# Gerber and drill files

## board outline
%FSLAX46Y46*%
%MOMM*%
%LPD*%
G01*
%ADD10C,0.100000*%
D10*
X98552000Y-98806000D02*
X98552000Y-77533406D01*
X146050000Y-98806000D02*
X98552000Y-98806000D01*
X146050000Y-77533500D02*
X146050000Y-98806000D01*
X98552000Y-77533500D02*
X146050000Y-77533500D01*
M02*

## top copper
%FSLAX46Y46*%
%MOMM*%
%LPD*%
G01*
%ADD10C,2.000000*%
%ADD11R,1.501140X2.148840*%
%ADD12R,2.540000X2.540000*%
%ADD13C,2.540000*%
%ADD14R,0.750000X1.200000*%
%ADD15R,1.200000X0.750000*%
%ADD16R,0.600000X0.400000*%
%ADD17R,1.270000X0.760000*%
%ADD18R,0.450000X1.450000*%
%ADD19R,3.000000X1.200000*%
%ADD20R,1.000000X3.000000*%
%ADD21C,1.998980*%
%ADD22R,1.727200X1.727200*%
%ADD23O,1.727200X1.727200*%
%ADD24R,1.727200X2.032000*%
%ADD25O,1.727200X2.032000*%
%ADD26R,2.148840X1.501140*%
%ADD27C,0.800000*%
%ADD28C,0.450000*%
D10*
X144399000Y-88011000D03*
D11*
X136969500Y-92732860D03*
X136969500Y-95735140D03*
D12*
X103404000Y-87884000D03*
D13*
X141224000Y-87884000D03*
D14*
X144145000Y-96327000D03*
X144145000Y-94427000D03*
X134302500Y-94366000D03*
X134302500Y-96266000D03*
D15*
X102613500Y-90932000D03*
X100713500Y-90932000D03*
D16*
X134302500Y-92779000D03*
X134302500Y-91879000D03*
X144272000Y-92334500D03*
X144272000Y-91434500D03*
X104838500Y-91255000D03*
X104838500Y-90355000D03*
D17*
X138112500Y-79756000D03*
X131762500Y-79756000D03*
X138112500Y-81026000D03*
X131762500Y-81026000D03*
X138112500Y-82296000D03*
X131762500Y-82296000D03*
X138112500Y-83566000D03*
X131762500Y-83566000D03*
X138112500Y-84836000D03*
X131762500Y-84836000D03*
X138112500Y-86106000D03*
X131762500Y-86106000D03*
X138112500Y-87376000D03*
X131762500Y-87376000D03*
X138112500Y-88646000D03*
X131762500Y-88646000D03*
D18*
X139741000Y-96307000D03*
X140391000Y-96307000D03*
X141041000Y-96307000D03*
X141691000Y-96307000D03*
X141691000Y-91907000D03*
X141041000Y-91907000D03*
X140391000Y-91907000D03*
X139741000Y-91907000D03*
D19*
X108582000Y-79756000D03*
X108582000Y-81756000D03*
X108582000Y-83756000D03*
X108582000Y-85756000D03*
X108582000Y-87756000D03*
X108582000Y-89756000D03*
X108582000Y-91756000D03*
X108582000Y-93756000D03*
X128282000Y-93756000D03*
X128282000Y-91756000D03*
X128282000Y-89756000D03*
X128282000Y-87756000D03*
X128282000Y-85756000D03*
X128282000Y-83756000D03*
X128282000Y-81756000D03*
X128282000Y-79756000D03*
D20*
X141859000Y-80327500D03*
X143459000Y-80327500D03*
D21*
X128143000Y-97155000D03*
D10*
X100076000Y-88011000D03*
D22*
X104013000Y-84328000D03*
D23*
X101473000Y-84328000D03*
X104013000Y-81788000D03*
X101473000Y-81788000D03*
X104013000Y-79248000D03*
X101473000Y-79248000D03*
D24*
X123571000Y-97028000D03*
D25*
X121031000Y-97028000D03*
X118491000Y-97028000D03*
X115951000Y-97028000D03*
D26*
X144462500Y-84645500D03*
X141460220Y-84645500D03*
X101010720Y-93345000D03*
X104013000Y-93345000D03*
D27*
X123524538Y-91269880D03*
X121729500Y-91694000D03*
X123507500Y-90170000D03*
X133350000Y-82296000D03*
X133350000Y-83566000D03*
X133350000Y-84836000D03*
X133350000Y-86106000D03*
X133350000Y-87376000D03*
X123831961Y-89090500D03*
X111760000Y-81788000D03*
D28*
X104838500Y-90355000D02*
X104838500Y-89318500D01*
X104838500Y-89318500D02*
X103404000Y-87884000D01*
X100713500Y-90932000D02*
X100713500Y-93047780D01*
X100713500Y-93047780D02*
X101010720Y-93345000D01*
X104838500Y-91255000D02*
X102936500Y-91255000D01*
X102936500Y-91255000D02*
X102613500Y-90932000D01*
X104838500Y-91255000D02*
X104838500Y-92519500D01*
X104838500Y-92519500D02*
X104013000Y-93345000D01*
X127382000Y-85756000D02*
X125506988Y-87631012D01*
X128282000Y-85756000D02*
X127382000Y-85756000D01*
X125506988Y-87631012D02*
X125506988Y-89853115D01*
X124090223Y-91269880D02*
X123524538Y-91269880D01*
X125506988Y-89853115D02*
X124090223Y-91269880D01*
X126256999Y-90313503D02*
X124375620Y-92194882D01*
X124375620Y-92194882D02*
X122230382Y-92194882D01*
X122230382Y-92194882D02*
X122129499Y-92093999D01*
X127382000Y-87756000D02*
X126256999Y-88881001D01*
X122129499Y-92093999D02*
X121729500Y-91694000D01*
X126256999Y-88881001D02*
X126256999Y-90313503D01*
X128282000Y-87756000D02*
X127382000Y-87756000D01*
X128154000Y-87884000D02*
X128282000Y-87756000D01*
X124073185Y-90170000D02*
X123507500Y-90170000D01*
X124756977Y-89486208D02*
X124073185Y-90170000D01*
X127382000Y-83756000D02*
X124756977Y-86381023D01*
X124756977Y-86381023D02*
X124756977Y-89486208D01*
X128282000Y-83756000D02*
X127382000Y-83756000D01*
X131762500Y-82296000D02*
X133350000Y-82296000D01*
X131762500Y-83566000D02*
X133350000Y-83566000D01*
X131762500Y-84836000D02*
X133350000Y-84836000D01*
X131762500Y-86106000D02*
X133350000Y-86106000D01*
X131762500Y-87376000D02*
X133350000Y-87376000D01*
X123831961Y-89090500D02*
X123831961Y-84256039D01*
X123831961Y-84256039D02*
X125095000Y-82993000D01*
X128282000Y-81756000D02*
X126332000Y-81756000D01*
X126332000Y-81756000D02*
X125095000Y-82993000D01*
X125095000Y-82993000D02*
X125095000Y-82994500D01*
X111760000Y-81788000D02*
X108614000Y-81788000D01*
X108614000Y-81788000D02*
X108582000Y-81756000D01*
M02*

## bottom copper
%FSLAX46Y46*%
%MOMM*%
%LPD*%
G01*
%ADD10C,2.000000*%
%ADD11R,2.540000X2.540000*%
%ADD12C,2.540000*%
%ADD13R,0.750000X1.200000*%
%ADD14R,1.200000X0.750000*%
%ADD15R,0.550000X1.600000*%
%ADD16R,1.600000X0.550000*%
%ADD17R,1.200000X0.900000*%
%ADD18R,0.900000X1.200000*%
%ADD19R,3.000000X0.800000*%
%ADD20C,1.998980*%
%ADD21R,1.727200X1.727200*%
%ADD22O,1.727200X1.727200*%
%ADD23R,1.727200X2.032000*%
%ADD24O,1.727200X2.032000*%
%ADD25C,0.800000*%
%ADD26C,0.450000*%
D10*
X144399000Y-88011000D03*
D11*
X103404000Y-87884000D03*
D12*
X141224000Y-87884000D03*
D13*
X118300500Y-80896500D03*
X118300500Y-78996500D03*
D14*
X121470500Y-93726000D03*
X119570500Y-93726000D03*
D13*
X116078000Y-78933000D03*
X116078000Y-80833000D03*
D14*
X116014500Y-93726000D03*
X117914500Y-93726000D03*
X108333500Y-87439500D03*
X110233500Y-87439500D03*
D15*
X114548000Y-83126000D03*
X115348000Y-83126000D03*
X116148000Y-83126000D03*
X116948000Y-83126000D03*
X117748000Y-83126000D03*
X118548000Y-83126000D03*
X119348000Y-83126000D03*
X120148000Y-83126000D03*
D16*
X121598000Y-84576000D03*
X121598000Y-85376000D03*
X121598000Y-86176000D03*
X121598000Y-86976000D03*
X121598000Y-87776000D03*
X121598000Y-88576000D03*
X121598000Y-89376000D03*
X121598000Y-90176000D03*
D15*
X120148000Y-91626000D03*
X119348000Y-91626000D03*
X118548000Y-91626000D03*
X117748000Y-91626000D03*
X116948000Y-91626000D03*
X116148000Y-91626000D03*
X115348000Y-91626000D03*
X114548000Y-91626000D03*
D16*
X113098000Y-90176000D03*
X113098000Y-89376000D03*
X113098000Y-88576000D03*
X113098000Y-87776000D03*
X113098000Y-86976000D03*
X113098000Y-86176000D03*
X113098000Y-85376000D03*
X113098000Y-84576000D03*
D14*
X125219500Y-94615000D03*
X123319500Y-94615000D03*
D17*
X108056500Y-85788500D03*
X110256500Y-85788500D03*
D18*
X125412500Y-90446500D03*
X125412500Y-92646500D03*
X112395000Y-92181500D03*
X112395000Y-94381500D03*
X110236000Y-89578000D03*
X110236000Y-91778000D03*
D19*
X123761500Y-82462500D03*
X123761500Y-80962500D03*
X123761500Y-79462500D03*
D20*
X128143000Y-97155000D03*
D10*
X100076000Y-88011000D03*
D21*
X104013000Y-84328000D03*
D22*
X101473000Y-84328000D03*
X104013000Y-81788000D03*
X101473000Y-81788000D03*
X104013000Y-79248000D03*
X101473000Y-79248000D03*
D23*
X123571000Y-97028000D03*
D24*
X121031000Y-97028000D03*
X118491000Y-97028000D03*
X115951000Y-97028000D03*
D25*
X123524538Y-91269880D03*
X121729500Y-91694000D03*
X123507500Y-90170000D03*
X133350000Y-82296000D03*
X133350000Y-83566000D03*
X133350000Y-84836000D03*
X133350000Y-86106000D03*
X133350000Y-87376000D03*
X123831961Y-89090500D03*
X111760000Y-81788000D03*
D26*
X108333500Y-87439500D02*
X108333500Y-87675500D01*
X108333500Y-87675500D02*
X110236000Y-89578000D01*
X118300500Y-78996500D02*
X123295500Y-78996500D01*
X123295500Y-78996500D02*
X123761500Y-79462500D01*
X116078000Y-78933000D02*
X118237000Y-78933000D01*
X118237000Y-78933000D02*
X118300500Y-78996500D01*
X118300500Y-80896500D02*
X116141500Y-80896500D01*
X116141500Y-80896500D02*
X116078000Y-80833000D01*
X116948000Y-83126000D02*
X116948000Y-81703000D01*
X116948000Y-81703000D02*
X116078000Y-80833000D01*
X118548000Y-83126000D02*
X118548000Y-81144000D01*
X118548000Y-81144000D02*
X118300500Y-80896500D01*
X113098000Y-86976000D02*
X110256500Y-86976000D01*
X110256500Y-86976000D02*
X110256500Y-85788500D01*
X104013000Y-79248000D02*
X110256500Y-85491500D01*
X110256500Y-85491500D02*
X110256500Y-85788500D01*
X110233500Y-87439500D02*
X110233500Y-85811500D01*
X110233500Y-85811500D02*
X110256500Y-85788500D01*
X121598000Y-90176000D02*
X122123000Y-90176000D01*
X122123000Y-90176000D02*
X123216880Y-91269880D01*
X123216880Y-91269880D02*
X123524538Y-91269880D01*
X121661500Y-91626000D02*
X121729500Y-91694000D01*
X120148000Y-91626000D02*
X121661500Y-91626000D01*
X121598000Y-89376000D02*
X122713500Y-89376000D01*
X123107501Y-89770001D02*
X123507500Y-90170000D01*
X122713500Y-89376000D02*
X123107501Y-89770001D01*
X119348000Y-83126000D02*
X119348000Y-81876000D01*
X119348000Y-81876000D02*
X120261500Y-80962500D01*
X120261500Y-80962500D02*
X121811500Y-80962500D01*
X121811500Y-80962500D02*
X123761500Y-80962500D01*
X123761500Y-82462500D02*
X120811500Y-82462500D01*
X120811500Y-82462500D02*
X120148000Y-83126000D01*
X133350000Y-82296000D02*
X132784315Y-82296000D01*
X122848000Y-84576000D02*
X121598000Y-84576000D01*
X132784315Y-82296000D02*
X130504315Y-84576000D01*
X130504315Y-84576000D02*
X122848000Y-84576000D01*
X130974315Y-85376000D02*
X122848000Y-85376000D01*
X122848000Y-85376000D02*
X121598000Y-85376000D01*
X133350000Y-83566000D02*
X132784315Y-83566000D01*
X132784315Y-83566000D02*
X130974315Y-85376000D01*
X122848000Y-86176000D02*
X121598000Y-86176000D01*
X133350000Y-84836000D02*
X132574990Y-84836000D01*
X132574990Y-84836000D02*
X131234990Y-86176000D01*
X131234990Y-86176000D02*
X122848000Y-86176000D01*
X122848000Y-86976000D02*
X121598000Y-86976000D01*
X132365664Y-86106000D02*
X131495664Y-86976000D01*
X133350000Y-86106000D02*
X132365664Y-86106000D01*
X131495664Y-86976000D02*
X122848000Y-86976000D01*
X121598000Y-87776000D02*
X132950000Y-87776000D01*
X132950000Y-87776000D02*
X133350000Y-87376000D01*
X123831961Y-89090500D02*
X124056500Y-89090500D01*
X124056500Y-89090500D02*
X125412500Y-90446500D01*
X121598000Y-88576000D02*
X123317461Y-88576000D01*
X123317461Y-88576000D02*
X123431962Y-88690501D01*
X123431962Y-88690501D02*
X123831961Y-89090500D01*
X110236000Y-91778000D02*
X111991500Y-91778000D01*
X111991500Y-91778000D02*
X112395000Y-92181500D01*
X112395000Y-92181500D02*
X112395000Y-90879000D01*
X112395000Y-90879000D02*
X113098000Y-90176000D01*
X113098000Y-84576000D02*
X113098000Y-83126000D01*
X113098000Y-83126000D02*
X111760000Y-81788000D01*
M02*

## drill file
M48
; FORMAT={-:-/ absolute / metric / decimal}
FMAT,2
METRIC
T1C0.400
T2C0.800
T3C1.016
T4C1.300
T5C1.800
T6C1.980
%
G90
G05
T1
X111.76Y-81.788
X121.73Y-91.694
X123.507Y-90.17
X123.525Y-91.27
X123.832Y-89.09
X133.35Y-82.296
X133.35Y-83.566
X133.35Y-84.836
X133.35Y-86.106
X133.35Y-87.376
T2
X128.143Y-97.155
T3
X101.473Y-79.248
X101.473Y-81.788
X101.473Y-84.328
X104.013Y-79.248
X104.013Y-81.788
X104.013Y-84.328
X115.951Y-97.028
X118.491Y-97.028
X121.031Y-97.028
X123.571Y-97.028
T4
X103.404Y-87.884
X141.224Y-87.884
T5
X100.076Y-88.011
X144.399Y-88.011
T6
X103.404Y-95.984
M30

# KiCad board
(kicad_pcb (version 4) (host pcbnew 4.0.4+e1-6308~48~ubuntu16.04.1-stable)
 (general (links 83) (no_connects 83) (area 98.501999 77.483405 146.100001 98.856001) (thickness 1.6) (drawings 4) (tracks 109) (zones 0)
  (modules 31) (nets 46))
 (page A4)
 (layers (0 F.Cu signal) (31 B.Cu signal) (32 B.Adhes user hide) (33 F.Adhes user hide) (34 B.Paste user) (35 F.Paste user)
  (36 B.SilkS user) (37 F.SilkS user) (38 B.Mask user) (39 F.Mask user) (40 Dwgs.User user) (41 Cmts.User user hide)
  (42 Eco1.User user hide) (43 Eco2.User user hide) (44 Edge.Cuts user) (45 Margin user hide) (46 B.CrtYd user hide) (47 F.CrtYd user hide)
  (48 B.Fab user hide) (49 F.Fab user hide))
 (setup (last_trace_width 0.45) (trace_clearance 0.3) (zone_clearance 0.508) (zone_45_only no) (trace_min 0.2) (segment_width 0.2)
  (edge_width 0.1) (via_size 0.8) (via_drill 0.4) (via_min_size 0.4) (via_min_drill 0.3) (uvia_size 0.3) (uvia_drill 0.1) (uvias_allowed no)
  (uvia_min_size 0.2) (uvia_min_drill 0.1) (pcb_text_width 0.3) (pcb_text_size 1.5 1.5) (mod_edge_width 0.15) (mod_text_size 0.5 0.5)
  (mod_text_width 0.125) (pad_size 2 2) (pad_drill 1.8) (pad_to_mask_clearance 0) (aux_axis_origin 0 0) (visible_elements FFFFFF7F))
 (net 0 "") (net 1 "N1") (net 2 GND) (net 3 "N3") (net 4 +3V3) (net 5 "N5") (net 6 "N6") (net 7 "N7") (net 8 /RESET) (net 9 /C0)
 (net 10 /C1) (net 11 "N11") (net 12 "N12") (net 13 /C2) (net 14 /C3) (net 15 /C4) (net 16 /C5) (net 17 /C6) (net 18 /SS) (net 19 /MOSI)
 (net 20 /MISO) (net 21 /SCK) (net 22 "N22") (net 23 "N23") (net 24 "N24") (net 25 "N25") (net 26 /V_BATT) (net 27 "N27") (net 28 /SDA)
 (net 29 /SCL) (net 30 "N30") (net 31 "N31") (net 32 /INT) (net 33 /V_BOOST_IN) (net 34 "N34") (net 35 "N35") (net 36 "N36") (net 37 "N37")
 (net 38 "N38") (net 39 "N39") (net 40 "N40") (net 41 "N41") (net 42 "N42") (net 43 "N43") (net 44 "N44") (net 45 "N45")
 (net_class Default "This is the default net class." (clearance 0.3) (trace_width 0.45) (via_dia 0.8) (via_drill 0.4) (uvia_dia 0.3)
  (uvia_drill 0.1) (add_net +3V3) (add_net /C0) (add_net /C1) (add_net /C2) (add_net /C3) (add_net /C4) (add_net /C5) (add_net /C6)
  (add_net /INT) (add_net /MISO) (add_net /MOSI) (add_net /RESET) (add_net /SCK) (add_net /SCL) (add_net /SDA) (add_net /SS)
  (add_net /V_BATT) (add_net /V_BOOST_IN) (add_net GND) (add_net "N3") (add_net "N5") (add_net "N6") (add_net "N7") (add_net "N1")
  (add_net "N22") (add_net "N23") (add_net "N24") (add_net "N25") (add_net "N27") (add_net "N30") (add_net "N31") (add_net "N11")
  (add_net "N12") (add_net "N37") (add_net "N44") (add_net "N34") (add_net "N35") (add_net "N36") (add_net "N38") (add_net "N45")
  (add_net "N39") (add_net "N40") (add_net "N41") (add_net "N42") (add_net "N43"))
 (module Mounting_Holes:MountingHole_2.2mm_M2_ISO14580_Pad (layer F.Cu) (at 144.399 88.011)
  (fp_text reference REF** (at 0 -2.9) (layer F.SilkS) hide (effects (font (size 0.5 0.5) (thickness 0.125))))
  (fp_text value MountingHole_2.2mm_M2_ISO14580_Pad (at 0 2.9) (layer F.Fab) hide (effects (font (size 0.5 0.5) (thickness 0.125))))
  (pad "" np_thru_hole circle (at 0 0) (size 2 2) (drill 1.8) (layers *.Cu) (zone_connect 0)))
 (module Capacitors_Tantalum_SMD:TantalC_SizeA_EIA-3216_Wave (layer F.Cu) (at 136.9695 94.234 90)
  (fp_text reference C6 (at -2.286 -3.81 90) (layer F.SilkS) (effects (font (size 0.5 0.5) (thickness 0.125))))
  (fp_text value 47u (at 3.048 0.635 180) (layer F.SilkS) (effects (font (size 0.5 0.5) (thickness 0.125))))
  (pad 2 smd rect (at 1.50114 0 90) (size 2.14884 1.50114) (layers F.Cu F.Paste F.Mask) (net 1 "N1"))
  (pad 1 smd rect (at -1.50114 0 90) (size 2.14884 1.50114) (layers F.Cu F.Paste F.Mask) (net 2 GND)))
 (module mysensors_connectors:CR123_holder (layer B.Cu) (at 103.404 87.884 270)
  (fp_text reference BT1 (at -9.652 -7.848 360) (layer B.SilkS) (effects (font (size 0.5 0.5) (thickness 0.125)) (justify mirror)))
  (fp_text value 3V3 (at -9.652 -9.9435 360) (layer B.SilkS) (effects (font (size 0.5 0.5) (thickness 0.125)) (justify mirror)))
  (pad 1 thru_hole rect (at 0 0 270) (size 2.54 2.54) (drill 1.3) (layers *.Cu *.Mask B.SilkS) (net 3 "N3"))
  (pad 2 thru_hole circle (at 0 -37.82 270) (size 2.54 2.54) (drill 1.3) (layers *.Cu *.Mask B.SilkS) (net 2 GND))
  (pad "" np_thru_hole circle (at 8.1 0 270) (size 1.98 1.98) (drill 1.98) (layers *.Cu Dwgs.User)))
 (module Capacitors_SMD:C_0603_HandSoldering (layer B.Cu) (at 118.3005 79.9465 90)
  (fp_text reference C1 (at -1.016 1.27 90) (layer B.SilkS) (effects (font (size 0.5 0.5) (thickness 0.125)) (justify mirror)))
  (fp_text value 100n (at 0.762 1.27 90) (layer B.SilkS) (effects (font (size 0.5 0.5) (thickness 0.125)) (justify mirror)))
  (pad 1 smd rect (at -0.95 0 90) (size 1.2 0.75) (layers B.Cu B.Paste B.Mask) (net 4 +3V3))
  (pad 2 smd rect (at 0.95 0 90) (size 1.2 0.75) (layers B.Cu B.Paste B.Mask) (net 2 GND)))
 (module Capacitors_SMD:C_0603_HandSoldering (layer B.Cu) (at 120.5205 93.726 180)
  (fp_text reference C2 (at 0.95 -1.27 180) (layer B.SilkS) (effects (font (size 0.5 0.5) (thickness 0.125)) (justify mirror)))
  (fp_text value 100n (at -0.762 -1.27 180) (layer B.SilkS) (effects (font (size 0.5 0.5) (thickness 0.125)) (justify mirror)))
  (pad 1 smd rect (at -0.95 0 180) (size 1.2 0.75) (layers B.Cu B.Paste B.Mask) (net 2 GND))
  (pad 2 smd rect (at 0.95 0 180) (size 1.2 0.75) (layers B.Cu B.Paste B.Mask) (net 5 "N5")))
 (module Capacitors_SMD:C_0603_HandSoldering (layer B.Cu) (at 116.078 79.883 270)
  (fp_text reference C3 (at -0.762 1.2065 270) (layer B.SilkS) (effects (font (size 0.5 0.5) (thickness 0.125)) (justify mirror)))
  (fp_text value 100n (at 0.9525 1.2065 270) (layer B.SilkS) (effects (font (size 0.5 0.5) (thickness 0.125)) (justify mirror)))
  (pad 1 smd rect (at -0.95 0 270) (size 1.2 0.75) (layers B.Cu B.Paste B.Mask) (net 2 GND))
  (pad 2 smd rect (at 0.95 0 270) (size 1.2 0.75) (layers B.Cu B.Paste B.Mask) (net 4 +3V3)))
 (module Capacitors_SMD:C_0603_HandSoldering (layer B.Cu) (at 116.9645 93.726)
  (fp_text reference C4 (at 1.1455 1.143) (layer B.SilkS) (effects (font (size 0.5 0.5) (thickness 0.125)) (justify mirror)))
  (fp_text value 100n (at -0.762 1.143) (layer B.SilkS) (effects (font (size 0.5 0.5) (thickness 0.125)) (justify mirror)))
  (pad 1 smd rect (at -0.95 0) (size 1.2 0.75) (layers B.Cu B.Paste B.Mask) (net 2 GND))
  (pad 2 smd rect (at 0.95 0) (size 1.2 0.75) (layers B.Cu B.Paste B.Mask) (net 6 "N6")))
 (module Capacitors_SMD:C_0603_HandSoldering (layer F.Cu) (at 144.145 95.377 90)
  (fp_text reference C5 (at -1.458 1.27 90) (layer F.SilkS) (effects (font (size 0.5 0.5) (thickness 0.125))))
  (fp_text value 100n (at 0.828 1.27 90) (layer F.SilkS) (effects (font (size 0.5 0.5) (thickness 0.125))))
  (pad 1 smd rect (at -0.95 0 90) (size 1.2 0.75) (layers F.Cu F.Paste F.Mask) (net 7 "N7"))
  (pad 2 smd rect (at 0.95 0 90) (size 1.2 0.75) (layers F.Cu F.Paste F.Mask) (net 2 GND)))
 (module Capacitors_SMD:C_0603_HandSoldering (layer B.Cu) (at 109.2835 87.4395)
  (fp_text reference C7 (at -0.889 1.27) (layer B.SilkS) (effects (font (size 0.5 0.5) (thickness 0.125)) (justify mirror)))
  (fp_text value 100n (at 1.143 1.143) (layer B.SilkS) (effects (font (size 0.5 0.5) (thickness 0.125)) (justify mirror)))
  (pad 1 smd rect (at -0.95 0) (size 1.2 0.75) (layers B.Cu B.Paste B.Mask) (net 2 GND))
  (pad 2 smd rect (at 0.95 0) (size 1.2 0.75) (layers B.Cu B.Paste B.Mask) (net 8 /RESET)))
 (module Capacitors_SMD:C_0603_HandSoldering (layer F.Cu) (at 134.3025 95.316 270)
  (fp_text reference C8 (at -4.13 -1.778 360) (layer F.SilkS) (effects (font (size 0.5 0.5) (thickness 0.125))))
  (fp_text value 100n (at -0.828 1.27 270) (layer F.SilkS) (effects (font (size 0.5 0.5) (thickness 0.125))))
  (pad 1 smd rect (at -0.95 0 270) (size 1.2 0.75) (layers F.Cu F.Paste F.Mask) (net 1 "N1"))
  (pad 2 smd rect (at 0.95 0 270) (size 1.2 0.75) (layers F.Cu F.Paste F.Mask) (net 2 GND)))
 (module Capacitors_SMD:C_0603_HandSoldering (layer F.Cu) (at 101.6635 90.932 180)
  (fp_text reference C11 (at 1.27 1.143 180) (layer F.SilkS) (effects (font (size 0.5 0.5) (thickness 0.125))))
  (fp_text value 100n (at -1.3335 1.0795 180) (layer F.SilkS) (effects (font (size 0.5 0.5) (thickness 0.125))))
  (pad 1 smd rect (at -0.95 0 180) (size 1.2 0.75) (layers F.Cu F.Paste F.Mask) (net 4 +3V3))
  (pad 2 smd rect (at 0.95 0 180) (size 1.2 0.75) (layers F.Cu F.Paste F.Mask) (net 2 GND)))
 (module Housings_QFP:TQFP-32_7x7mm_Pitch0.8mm (layer B.Cu) (at 117.348 87.376 270)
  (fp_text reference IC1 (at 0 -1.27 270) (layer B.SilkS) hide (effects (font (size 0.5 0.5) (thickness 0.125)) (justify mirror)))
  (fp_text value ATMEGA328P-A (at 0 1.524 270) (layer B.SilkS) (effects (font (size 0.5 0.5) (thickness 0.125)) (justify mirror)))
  (pad 1 smd rect (at -4.25 2.8 270) (size 1.6 0.55) (layers B.Cu B.Paste B.Mask) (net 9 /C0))
  (pad 2 smd rect (at -4.25 2 270) (size 1.6 0.55) (layers B.Cu B.Paste B.Mask) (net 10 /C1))
  (pad 3 smd rect (at -4.25 1.2 270) (size 1.6 0.55) (layers B.Cu B.Paste B.Mask) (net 2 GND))
  (pad 4 smd rect (at -4.25 0.4 270) (size 1.6 0.55) (layers B.Cu B.Paste B.Mask) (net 4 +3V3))
  (pad 5 smd rect (at -4.25 -0.4 270) (size 1.6 0.55) (layers B.Cu B.Paste B.Mask) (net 2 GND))
  (pad 6 smd rect (at -4.25 -1.2 270) (size 1.6 0.55) (layers B.Cu B.Paste B.Mask) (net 4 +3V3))
  (pad 7 smd rect (at -4.25 -2 270) (size 1.6 0.55) (layers B.Cu B.Paste B.Mask) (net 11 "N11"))
  (pad 8 smd rect (at -4.25 -2.8 270) (size 1.6 0.55) (layers B.Cu B.Paste B.Mask) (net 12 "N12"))
  (pad 9 smd rect (at -2.8 -4.25 180) (size 1.6 0.55) (layers B.Cu B.Paste B.Mask) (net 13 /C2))
  (pad 10 smd rect (at -2 -4.25 180) (size 1.6 0.55) (layers B.Cu B.Paste B.Mask) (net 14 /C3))
  (pad 11 smd rect (at -1.2 -4.25 180) (size 1.6 0.55) (layers B.Cu B.Paste B.Mask) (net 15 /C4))
  (pad 12 smd rect (at -0.4 -4.25 180) (size 1.6 0.55) (layers B.Cu B.Paste B.Mask) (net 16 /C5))
  (pad 13 smd rect (at 0.4 -4.25 180) (size 1.6 0.55) (layers B.Cu B.Paste B.Mask) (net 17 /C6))
  (pad 14 smd rect (at 1.2 -4.25 180) (size 1.6 0.55) (layers B.Cu B.Paste B.Mask) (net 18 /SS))
  (pad 15 smd rect (at 2 -4.25 180) (size 1.6 0.55) (layers B.Cu B.Paste B.Mask) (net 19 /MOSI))
  (pad 16 smd rect (at 2.8 -4.25 180) (size 1.6 0.55) (layers B.Cu B.Paste B.Mask) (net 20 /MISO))
  (pad 17 smd rect (at 4.25 -2.8 270) (size 1.6 0.55) (layers B.Cu B.Paste B.Mask) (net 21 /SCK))
  (pad 18 smd rect (at 4.25 -2 270) (size 1.6 0.55) (layers B.Cu B.Paste B.Mask) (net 5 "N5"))
  (pad 19 smd rect (at 4.25 -1.2 270) (size 1.6 0.55) (layers B.Cu B.Paste B.Mask) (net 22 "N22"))
  (pad 20 smd rect (at 4.25 -0.4 270) (size 1.6 0.55) (layers B.Cu B.Paste B.Mask) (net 6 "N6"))
  (pad 21 smd rect (at 4.25 0.4 270) (size 1.6 0.55) (layers B.Cu B.Paste B.Mask) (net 2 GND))
  (pad 22 smd rect (at 4.25 1.2 270) (size 1.6 0.55) (layers B.Cu B.Paste B.Mask) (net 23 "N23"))
  (pad 23 smd rect (at 4.25 2 270) (size 1.6 0.55) (layers B.Cu B.Paste B.Mask) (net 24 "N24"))
  (pad 24 smd rect (at 4.25 2.8 270) (size 1.6 0.55) (layers B.Cu B.Paste B.Mask) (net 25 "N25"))
  (pad 25 smd rect (at 2.8 4.25 180) (size 1.6 0.55) (layers B.Cu B.Paste B.Mask) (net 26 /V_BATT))
  (pad 26 smd rect (at 2 4.25 180) (size 1.6 0.55) (layers B.Cu B.Paste B.Mask) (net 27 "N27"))
  (pad 27 smd rect (at 1.2 4.25 180) (size 1.6 0.55) (layers B.Cu B.Paste B.Mask) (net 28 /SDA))
  (pad 28 smd rect (at 0.4 4.25 180) (size 1.6 0.55) (layers B.Cu B.Paste B.Mask) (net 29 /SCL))
  (pad 29 smd rect (at -0.4 4.25 180) (size 1.6 0.55) (layers B.Cu B.Paste B.Mask) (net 8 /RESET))
  (pad 30 smd rect (at -1.2 4.25 180) (size 1.6 0.55) (layers B.Cu B.Paste B.Mask) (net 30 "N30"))
  (pad 31 smd rect (at -2 4.25 180) (size 1.6 0.55) (layers B.Cu B.Paste B.Mask) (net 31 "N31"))
  (pad 32 smd rect (at -2.8 4.25 180) (size 1.6 0.55) (layers B.Cu B.Paste B.Mask) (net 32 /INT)))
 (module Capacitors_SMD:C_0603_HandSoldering (layer B.Cu) (at 124.2695 94.615 180)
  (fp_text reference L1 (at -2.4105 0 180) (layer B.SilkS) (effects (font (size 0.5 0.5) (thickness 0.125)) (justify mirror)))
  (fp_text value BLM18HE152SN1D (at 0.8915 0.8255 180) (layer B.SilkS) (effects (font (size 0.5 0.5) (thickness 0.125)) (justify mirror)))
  (pad 1 smd rect (at -0.95 0 180) (size 1.2 0.75) (layers B.Cu B.Paste B.Mask) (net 4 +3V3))
  (pad 2 smd rect (at 0.95 0 180) (size 1.2 0.75) (layers B.Cu B.Paste B.Mask) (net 5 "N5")))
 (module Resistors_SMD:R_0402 (layer F.Cu) (at 134.3025 92.329 90)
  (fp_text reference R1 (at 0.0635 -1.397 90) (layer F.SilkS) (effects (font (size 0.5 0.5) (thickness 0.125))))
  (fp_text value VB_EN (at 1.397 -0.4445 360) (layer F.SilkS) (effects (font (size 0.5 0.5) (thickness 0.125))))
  (pad 1 smd rect (at -0.45 0 90) (size 0.4 0.6) (layers F.Cu F.Paste F.Mask) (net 1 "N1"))
  (pad 2 smd rect (at 0.45 0 90) (size 0.4 0.6) (layers F.Cu F.Paste F.Mask) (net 4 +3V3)))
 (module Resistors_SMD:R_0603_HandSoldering (layer B.Cu) (at 109.1565 85.7885)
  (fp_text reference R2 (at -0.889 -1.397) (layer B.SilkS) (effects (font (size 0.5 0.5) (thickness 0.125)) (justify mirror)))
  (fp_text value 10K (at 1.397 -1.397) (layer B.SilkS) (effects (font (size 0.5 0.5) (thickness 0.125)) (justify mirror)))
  (pad 1 smd rect (at -1.1 0) (size 1.2 0.9) (layers B.Cu B.Paste B.Mask) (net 4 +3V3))
  (pad 2 smd rect (at 1.1 0) (size 1.2 0.9) (layers B.Cu B.Paste B.Mask) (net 8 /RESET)))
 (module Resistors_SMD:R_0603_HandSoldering (layer B.Cu) (at 125.4125 91.5465 270)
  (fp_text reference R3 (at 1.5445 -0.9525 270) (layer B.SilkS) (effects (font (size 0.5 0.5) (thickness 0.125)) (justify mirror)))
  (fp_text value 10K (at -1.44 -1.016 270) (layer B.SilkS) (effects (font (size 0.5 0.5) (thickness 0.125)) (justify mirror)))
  (pad 1 smd rect (at -1.1 0 270) (size 1.2 0.9) (layers B.Cu B.Paste B.Mask) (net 18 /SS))
  (pad 2 smd rect (at 1.1 0 270) (size 1.2 0.9) (layers B.Cu B.Paste B.Mask) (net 4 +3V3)))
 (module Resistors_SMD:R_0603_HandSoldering (layer B.Cu) (at 112.395 93.2815 270)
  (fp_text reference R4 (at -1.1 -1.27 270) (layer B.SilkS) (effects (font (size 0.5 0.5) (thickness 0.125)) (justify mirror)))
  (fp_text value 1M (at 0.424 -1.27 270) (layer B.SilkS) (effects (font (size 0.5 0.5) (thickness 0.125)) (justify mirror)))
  (pad 1 smd rect (at -1.1 0 270) (size 1.2 0.9) (layers B.Cu B.Paste B.Mask) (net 26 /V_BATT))
  (pad 2 smd rect (at 1.1 0 270) (size 1.2 0.9) (layers B.Cu B.Paste B.Mask) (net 3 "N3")))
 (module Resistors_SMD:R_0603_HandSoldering (layer B.Cu) (at 110.236 90.678 270)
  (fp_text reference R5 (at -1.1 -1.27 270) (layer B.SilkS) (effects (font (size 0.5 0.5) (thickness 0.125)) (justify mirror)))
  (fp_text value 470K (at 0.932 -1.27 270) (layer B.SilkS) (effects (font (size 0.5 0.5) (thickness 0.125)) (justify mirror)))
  (pad 1 smd rect (at -1.1 0 270) (size 1.2 0.9) (layers B.Cu B.Paste B.Mask) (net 2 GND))
  (pad 2 smd rect (at 1.1 0 270) (size 1.2 0.9) (layers B.Cu B.Paste B.Mask) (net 26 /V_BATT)))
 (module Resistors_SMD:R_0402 (layer F.Cu) (at 144.272 91.8845 90)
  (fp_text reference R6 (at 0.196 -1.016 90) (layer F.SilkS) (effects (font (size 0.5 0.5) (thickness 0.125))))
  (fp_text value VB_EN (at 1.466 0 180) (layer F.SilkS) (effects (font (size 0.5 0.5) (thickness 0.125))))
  (pad 1 smd rect (at -0.45 0 90) (size 0.4 0.6) (layers F.Cu F.Paste F.Mask) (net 3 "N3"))
  (pad 2 smd rect (at 0.45 0 90) (size 0.4 0.6) (layers F.Cu F.Paste F.Mask) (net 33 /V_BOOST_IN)))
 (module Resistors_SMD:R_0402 (layer F.Cu) (at 104.8385 90.805 90)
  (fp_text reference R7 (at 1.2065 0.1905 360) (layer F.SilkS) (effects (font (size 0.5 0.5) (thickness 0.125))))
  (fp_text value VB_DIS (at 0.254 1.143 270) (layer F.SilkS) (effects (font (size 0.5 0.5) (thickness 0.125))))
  (pad 1 smd rect (at -0.45 0 90) (size 0.4 0.6) (layers F.Cu F.Paste F.Mask) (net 4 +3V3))
  (pad 2 smd rect (at 0.45 0 90) (size 0.4 0.6) (layers F.Cu F.Paste F.Mask) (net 3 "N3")))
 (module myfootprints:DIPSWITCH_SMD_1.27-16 (layer F.Cu) (at 134.9375 84.201 270)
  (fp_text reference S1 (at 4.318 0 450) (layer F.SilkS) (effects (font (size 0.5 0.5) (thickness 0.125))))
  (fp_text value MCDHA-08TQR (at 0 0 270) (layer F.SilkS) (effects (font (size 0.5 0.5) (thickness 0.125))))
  (pad 16 smd rect (at -4.445 -3.175 270) (size 0.76 1.27) (layers F.Cu F.Paste F.Mask) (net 2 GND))
  (pad 1 smd rect (at -4.445 3.175 270) (size 0.76 1.27) (layers F.Cu F.Paste F.Mask) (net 9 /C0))
  (pad 15 smd rect (at -3.175 -3.175 270) (size 0.76 1.27) (layers F.Cu F.Paste F.Mask) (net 2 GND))
  (pad 2 smd rect (at -3.175 3.175 270) (size 0.76 1.27) (layers F.Cu F.Paste F.Mask) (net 10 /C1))
  (pad 14 smd rect (at -1.905 -3.175 270) (size 0.76 1.27) (layers F.Cu F.Paste F.Mask) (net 2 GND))
  (pad 3 smd rect (at -1.905 3.175 270) (size 0.76 1.27) (layers F.Cu F.Paste F.Mask) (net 13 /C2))
  (pad 13 smd rect (at -0.635 -3.175 270) (size 0.76 1.27) (layers F.Cu F.Paste F.Mask) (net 2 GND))
  (pad 4 smd rect (at -0.635 3.175 270) (size 0.76 1.27) (layers F.Cu F.Paste F.Mask) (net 14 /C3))
  (pad 12 smd rect (at 0.635 -3.175 270) (size 0.76 1.27) (layers F.Cu F.Paste F.Mask) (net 2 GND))
  (pad 5 smd rect (at 0.635 3.175 270) (size 0.76 1.27) (layers F.Cu F.Paste F.Mask) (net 15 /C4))
  (pad 11 smd rect (at 1.905 -3.175 270) (size 0.76 1.27) (layers F.Cu F.Paste F.Mask) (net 2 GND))
  (pad 6 smd rect (at 1.905 3.175 270) (size 0.76 1.27) (layers F.Cu F.Paste F.Mask) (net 16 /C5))
  (pad 10 smd rect (at 3.175 -3.175 270) (size 0.76 1.27) (layers F.Cu F.Paste F.Mask) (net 2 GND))
  (pad 7 smd rect (at 3.175 3.175 270) (size 0.76 1.27) (layers F.Cu F.Paste F.Mask) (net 17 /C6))
  (pad 9 smd rect (at 4.445 -3.175 270) (size 0.76 1.27) (layers F.Cu F.Paste F.Mask) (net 2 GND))
  (pad 8 smd rect (at 4.445 3.175 270) (size 0.76 1.27) (layers F.Cu F.Paste F.Mask) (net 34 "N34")))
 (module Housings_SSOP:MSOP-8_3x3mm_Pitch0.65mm (layer F.Cu) (at 140.716 94.107 90)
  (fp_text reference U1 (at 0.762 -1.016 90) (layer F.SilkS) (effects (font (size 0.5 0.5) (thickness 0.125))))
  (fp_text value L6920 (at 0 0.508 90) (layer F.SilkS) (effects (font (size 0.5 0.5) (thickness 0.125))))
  (pad 1 smd rect (at -2.2 -0.975 90) (size 1.45 0.45) (layers F.Cu F.Paste F.Mask) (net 1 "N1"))
  (pad 2 smd rect (at -2.2 -0.325 90) (size 1.45 0.45) (layers F.Cu F.Paste F.Mask) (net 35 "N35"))
  (pad 3 smd rect (at -2.2 0.325 90) (size 1.45 0.45) (layers F.Cu F.Paste F.Mask) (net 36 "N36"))
  (pad 4 smd rect (at -2.2 0.975 90) (size 1.45 0.45) (layers F.Cu F.Paste F.Mask) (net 7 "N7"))
  (pad 5 smd rect (at 2.2 0.975 90) (size 1.45 0.45) (layers F.Cu F.Paste F.Mask) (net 1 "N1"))
  (pad 6 smd rect (at 2.2 0.325 90) (size 1.45 0.45) (layers F.Cu F.Paste F.Mask) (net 2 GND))
  (pad 7 smd rect (at 2.2 -0.325 90) (size 1.45 0.45) (layers F.Cu F.Paste F.Mask) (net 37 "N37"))
  (pad 8 smd rect (at 2.2 -0.975 90) (size 1.45 0.45) (layers F.Cu F.Paste F.Mask) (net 1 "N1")))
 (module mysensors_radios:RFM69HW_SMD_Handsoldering (layer F.Cu) (at 109.982 79.756)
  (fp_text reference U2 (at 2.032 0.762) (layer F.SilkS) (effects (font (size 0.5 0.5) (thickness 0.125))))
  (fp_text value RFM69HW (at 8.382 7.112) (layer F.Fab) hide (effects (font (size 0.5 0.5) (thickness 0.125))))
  (pad 1 smd rect (at -1.4 0) (size 3 1.2) (layers F.Cu F.Paste F.Mask) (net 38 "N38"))
  (pad 2 smd rect (at -1.4 2) (size 3 1.2) (layers F.Cu F.Paste F.Mask) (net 32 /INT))
  (pad 3 smd rect (at -1.4 4) (size 3 1.2) (layers F.Cu F.Paste F.Mask) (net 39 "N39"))
  (pad 4 smd rect (at -1.4 6) (size 3 1.2) (layers F.Cu F.Paste F.Mask) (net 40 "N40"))
  (pad 5 smd rect (at -1.4 8) (size 3 1.2) (layers F.Cu F.Paste F.Mask) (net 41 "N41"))
  (pad 6 smd rect (at -1.4 10) (size 3 1.2) (layers F.Cu F.Paste F.Mask) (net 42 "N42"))
  (pad 7 smd rect (at -1.4 12) (size 3 1.2) (layers F.Cu F.Paste F.Mask) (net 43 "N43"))
  (pad 8 smd rect (at -1.4 14) (size 3 1.2) (layers F.Cu F.Paste F.Mask) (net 4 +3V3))
  (pad 9 smd rect (at 18.3 14) (size 3 1.2) (layers F.Cu F.Paste F.Mask) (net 2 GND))
  (pad 10 smd rect (at 18.3 12) (size 3 1.2) (layers F.Cu F.Paste F.Mask) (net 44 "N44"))
  (pad 11 smd rect (at 18.3 10) (size 3 1.2) (layers F.Cu F.Paste F.Mask) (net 2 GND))
  (pad 12 smd rect (at 18.3 8) (size 3 1.2) (layers F.Cu F.Paste F.Mask) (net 21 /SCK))
  (pad 13 smd rect (at 18.3 6) (size 3 1.2) (layers F.Cu F.Paste F.Mask) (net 20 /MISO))
  (pad 14 smd rect (at 18.3 4) (size 3 1.2) (layers F.Cu F.Paste F.Mask) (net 19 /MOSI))
  (pad 15 smd rect (at 18.3 2) (size 3 1.2) (layers F.Cu F.Paste F.Mask) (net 18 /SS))
  (pad 16 smd rect (at 18.3 0) (size 3 1.2) (layers F.Cu F.Paste F.Mask) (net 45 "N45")))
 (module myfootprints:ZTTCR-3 (layer B.Cu) (at 123.7615 80.9625 90)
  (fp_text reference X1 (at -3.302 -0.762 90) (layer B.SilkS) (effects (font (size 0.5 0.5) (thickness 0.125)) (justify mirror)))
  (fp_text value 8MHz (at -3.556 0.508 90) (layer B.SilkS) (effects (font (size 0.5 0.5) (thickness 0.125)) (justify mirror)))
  (pad 1 smd rect (at -1.5 0 90) (size 0.8 3) (layers B.Cu B.Paste B.Mask) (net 12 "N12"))
  (pad 2 smd rect (at 0 0 90) (size 0.8 3) (layers B.Cu B.Paste B.Mask) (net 11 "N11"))
  (pad 3 smd rect (at 1.5 0 90) (size 0.8 3) (layers B.Cu B.Paste B.Mask) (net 2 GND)))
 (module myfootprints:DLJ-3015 (layer F.Cu) (at 142.659 80.3275)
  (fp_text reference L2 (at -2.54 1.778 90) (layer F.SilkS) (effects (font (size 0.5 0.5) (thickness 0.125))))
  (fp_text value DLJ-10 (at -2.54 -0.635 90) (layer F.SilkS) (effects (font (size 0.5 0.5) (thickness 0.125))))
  (pad 1 smd rect (at -0.8 0) (size 1 3) (layers F.Cu F.Paste F.Mask) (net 37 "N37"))
  (pad 2 smd rect (at 0.8 0) (size 1 3) (layers F.Cu F.Paste F.Mask) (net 33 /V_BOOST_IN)))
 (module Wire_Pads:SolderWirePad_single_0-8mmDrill (layer F.Cu) (at 128.143 97.155)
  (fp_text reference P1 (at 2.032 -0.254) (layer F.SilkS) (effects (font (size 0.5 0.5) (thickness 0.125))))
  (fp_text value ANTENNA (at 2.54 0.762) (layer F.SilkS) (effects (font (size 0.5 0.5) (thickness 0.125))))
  (pad 1 thru_hole circle (at 0 0) (size 1.99898 1.99898) (drill 0.8001) (layers *.Cu *.Mask F.SilkS) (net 44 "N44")))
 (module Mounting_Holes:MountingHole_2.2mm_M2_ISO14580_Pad (layer F.Cu) (at 100.076 88.011)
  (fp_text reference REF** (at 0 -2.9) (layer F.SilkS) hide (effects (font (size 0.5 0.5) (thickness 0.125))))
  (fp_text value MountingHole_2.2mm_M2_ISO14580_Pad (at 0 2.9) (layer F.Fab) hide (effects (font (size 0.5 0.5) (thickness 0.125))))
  (pad "" np_thru_hole circle (at 0 0) (size 2 2) (drill 1.8) (layers *.Cu) (zone_connect 0)))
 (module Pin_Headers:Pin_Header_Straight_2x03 (layer F.Cu) (at 104.013 84.328 180)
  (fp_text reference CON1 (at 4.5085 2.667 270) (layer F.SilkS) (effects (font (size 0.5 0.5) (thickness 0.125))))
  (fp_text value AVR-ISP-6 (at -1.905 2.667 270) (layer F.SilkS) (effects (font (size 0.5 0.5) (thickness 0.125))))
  (pad 1 thru_hole rect (at 0 0 180) (size 1.7272 1.7272) (drill 1.016) (layers *.Cu *.Mask F.SilkS) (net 20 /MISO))
  (pad 2 thru_hole oval (at 2.54 0 180) (size 1.7272 1.7272) (drill 1.016) (layers *.Cu *.Mask F.SilkS) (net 4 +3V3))
  (pad 3 thru_hole oval (at 0 2.54 180) (size 1.7272 1.7272) (drill 1.016) (layers *.Cu *.Mask F.SilkS) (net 21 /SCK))
  (pad 4 thru_hole oval (at 2.54 2.54 180) (size 1.7272 1.7272) (drill 1.016) (layers *.Cu *.Mask F.SilkS) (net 19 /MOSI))
  (pad 5 thru_hole oval (at 0 5.08 180) (size 1.7272 1.7272) (drill 1.016) (layers *.Cu *.Mask F.SilkS) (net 8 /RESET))
  (pad 6 thru_hole oval (at 2.54 5.08 180) (size 1.7272 1.7272) (drill 1.016) (layers *.Cu *.Mask F.SilkS) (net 2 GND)))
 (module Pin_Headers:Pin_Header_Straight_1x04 (layer F.Cu) (at 123.571 97.028 270)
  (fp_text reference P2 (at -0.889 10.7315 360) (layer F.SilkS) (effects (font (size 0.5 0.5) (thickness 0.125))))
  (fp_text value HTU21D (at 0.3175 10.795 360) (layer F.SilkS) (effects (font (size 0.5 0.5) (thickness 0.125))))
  (pad 1 thru_hole rect (at 0 0 270) (size 2.032 1.7272) (drill 1.016) (layers *.Cu *.Mask F.SilkS) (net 4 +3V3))
  (pad 2 thru_hole oval (at 0 2.54 270) (size 2.032 1.7272) (drill 1.016) (layers *.Cu *.Mask F.SilkS) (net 2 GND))
  (pad 3 thru_hole oval (at 0 5.08 270) (size 2.032 1.7272) (drill 1.016) (layers *.Cu *.Mask F.SilkS) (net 28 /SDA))
  (pad 4 thru_hole oval (at 0 7.62 270) (size 2.032 1.7272) (drill 1.016) (layers *.Cu *.Mask F.SilkS) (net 29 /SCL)))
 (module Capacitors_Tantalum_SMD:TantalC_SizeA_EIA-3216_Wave (layer F.Cu) (at 142.96136 84.6455)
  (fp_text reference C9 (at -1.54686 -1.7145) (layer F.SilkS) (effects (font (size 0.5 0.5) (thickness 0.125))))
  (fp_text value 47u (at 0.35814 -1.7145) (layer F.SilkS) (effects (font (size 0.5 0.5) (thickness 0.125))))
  (pad 2 smd rect (at 1.50114 0) (size 2.14884 1.50114) (layers F.Cu F.Paste F.Mask) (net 33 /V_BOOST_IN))
  (pad 1 smd rect (at -1.50114 0) (size 2.14884 1.50114) (layers F.Cu F.Paste F.Mask) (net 2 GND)))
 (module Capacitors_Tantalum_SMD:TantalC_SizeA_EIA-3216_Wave (layer F.Cu) (at 102.51186 93.345 180)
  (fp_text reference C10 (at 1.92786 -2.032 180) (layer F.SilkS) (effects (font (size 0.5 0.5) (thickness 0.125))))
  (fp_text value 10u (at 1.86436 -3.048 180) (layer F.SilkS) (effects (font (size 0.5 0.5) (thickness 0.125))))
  (pad 2 smd rect (at 1.50114 0 180) (size 2.14884 1.50114) (layers F.Cu F.Paste F.Mask) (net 2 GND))
  (pad 1 smd rect (at -1.50114 0 180) (size 2.14884 1.50114) (layers F.Cu F.Paste F.Mask) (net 4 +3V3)))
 (gr_line (start 98.552 98.806) (end 98.552 77.533406) (layer Edge.Cuts) (width 0.1))
 (gr_line (start 146.05 98.806) (end 98.552 98.806) (layer Edge.Cuts) (width 0.1))
 (gr_line (start 146.05 77.5335) (end 146.05 98.806) (layer Edge.Cuts) (width 0.1))
 (gr_line (start 98.552 77.5335) (end 146.05 77.5335) (layer Edge.Cuts) (width 0.1))
 (segment (start 104.8385 90.355) (end 104.8385 89.3185) (width 0.45) (layer F.Cu) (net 3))
 (segment (start 104.8385 89.3185) (end 103.404 87.884) (width 0.45) (layer F.Cu) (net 3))
 (segment (start 100.7135 90.932) (end 100.7135 93.04778) (width 0.45) (layer F.Cu) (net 2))
 (segment (start 100.7135 93.04778) (end 101.01072 93.345) (width 0.45) (layer F.Cu) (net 2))
 (segment (start 108.3335 87.4395) (end 108.3335 87.6755) (width 0.45) (layer B.Cu) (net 2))
 (segment (start 108.3335 87.6755) (end 110.236 89.578) (width 0.45) (layer B.Cu) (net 2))
 (segment (start 118.3005 78.9965) (end 123.2955 78.9965) (width 0.45) (layer B.Cu) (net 2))
 (segment (start 123.2955 78.9965) (end 123.7615 79.4625) (width 0.45) (layer B.Cu) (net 2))
 (segment (start 116.078 78.933) (end 118.237 78.933) (width 0.45) (layer B.Cu) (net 2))
 (segment (start 118.237 78.933) (end 118.3005 78.9965) (width 0.45) (layer B.Cu) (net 2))
 (segment (start 104.8385 91.255) (end 102.9365 91.255) (width 0.45) (layer F.Cu) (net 4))
 (segment (start 102.9365 91.255) (end 102.6135 90.932) (width 0.45) (layer F.Cu) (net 4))
 (segment (start 104.8385 91.255) (end 104.8385 92.5195) (width 0.45) (layer F.Cu) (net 4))
 (segment (start 104.8385 92.5195) (end 104.013 93.345) (width 0.45) (layer F.Cu) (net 4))
 (segment (start 118.3005 80.8965) (end 116.1415 80.8965) (width 0.45) (layer B.Cu) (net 4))
 (segment (start 116.1415 80.8965) (end 116.078 80.833) (width 0.45) (layer B.Cu) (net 4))
 (segment (start 116.948 83.126) (end 116.948 81.703) (width 0.45) (layer B.Cu) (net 4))
 (segment (start 116.948 81.703) (end 116.078 80.833) (width 0.45) (layer B.Cu) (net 4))
 (segment (start 118.548 83.126) (end 118.548 81.144) (width 0.45) (layer B.Cu) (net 4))
 (segment (start 118.548 81.144) (end 118.3005 80.8965) (width 0.45) (layer B.Cu) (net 4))
 (segment (start 113.098 86.976) (end 110.2565 86.976) (width 0.45) (layer B.Cu) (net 8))
 (segment (start 110.2565 86.976) (end 110.2565 85.7885) (width 0.45) (layer B.Cu) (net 8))
 (segment (start 104.013 79.248) (end 110.2565 85.4915) (width 0.45) (layer B.Cu) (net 8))
 (segment (start 110.2565 85.4915) (end 110.2565 85.7885) (width 0.45) (layer B.Cu) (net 8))
 (segment (start 110.2335 87.4395) (end 110.2335 85.8115) (width 0.45) (layer B.Cu) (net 8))
 (segment (start 110.2335 85.8115) (end 110.2565 85.7885) (width 0.45) (layer B.Cu) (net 8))
 (segment (start 127.382 85.756) (end 125.506988 87.631012) (width 0.45) (layer F.Cu) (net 20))
 (segment (start 128.282 85.756) (end 127.382 85.756) (width 0.45) (layer F.Cu) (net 20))
 (segment (start 125.506988 87.631012) (end 125.506988 89.853115) (width 0.45) (layer F.Cu) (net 20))
 (segment (start 124.090223 91.26988) (end 123.524538 91.26988) (width 0.45) (layer F.Cu) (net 20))
 (segment (start 125.506988 89.853115) (end 124.090223 91.26988) (width 0.45) (layer F.Cu) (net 20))
 (segment (start 121.598 90.176) (end 122.123 90.176) (width 0.45) (layer B.Cu) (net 20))
 (via (at 123.524538 91.26988) (size 0.8) (drill 0.4) (layers F.Cu B.Cu) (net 20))
 (segment (start 122.123 90.176) (end 123.21688 91.26988) (width 0.45) (layer B.Cu) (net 20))
 (segment (start 123.21688 91.26988) (end 123.524538 91.26988) (width 0.45) (layer B.Cu) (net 20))
 (segment (start 126.256999 90.313503) (end 124.37562 92.194882) (width 0.45) (layer F.Cu) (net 21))
 (segment (start 124.37562 92.194882) (end 122.230382 92.194882) (width 0.45) (layer F.Cu) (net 21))
 (segment (start 122.230382 92.194882) (end 122.129499 92.093999) (width 0.45) (layer F.Cu) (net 21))
 (segment (start 127.382 87.756) (end 126.256999 88.881001) (width 0.45) (layer F.Cu) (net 21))
 (segment (start 122.129499 92.093999) (end 121.7295 91.694) (width 0.45) (layer F.Cu) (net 21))
 (segment (start 126.256999 88.881001) (end 126.256999 90.313503) (width 0.45) (layer F.Cu) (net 21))
 (segment (start 128.282 87.756) (end 127.382 87.756) (width 0.45) (layer F.Cu) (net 21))
 (segment (start 121.6615 91.626) (end 121.7295 91.694) (width 0.45) (layer B.Cu) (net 21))
 (segment (start 120.148 91.626) (end 121.6615 91.626) (width 0.45) (layer B.Cu) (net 21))
 (via (at 121.7295 91.694) (size 0.8) (drill 0.4) (layers F.Cu B.Cu) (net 21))
 (segment (start 128.154 87.884) (end 128.282 87.756) (width 0.45) (layer F.Cu) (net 21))
 (segment (start 124.073185 90.17) (end 123.5075 90.17) (width 0.45) (layer F.Cu) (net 19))
 (segment (start 124.756977 89.486208) (end 124.073185 90.17) (width 0.45) (layer F.Cu) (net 19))
 (segment (start 127.382 83.756) (end 124.756977 86.381023) (width 0.45) (layer F.Cu) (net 19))
 (segment (start 124.756977 86.381023) (end 124.756977 89.486208) (width 0.45) (layer F.Cu) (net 19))
 (segment (start 128.282 83.756) (end 127.382 83.756) (width 0.45) (layer F.Cu) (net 19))
 (segment (start 121.598 89.376) (end 122.7135 89.376) (width 0.45) (layer B.Cu) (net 19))
 (segment (start 123.107501 89.770001) (end 123.5075 90.17) (width 0.45) (layer B.Cu) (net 19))
 (segment (start 122.7135 89.376) (end 123.107501 89.770001) (width 0.45) (layer B.Cu) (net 19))
 (via (at 123.5075 90.17) (size 0.8) (drill 0.4) (layers F.Cu B.Cu) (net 19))
 (segment (start 119.348 83.126) (end 119.348 81.876) (width 0.45) (layer B.Cu) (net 11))
 (segment (start 119.348 81.876) (end 120.2615 80.9625) (width 0.45) (layer B.Cu) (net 11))
 (segment (start 120.2615 80.9625) (end 121.8115 80.9625) (width 0.45) (layer B.Cu) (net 11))
 (segment (start 121.8115 80.9625) (end 123.7615 80.9625) (width 0.45) (layer B.Cu) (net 11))
 (segment (start 123.7615 82.4625) (end 120.8115 82.4625) (width 0.45) (layer B.Cu) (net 12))
 (segment (start 120.8115 82.4625) (end 120.148 83.126) (width 0.45) (layer B.Cu) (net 12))
 (segment (start 133.35 82.296) (end 132.784315 82.296) (width 0.45) (layer B.Cu) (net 13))
 (segment (start 122.848 84.576) (end 121.598 84.576) (width 0.45) (layer B.Cu) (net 13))
 (segment (start 132.784315 82.296) (end 130.504315 84.576) (width 0.45) (layer B.Cu) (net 13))
 (segment (start 130.504315 84.576) (end 122.848 84.576) (width 0.45) (layer B.Cu) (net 13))
 (segment (start 131.7625 82.296) (end 133.35 82.296) (width 0.45) (layer F.Cu) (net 13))
 (via (at 133.35 82.296) (size 0.8) (drill 0.4) (layers F.Cu B.Cu) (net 13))
 (segment (start 130.974315 85.376) (end 122.848 85.376) (width 0.45) (layer B.Cu) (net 14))
 (segment (start 122.848 85.376) (end 121.598 85.376) (width 0.45) (layer B.Cu) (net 14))
 (segment (start 133.35 83.566) (end 132.784315 83.566) (width 0.45) (layer B.Cu) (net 14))
 (segment (start 132.784315 83.566) (end 130.974315 85.376) (width 0.45) (layer B.Cu) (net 14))
 (segment (start 131.7625 83.566) (end 133.35 83.566) (width 0.45) (layer F.Cu) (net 14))
 (via (at 133.35 83.566) (size 0.8) (drill 0.4) (layers F.Cu B.Cu) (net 14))
 (segment (start 122.848 86.176) (end 121.598 86.176) (width 0.45) (layer B.Cu) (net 15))
 (segment (start 133.35 84.836) (end 132.57499 84.836) (width 0.45) (layer B.Cu) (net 15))
 (segment (start 132.57499 84.836) (end 131.23499 86.176) (width 0.45) (layer B.Cu) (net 15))
 (segment (start 131.23499 86.176) (end 122.848 86.176) (width 0.45) (layer B.Cu) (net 15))
 (segment (start 131.7625 84.836) (end 133.35 84.836) (width 0.45) (layer F.Cu) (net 15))
 (via (at 133.35 84.836) (size 0.8) (drill 0.4) (layers F.Cu B.Cu) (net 15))
 (segment (start 122.848 86.976) (end 121.598 86.976) (width 0.45) (layer B.Cu) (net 16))
 (segment (start 132.365664 86.106) (end 131.495664 86.976) (width 0.45) (layer B.Cu) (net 16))
 (segment (start 133.35 86.106) (end 132.365664 86.106) (width 0.45) (layer B.Cu) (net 16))
 (segment (start 131.495664 86.976) (end 122.848 86.976) (width 0.45) (layer B.Cu) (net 16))
 (segment (start 131.7625 86.106) (end 133.35 86.106) (width 0.45) (layer F.Cu) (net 16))
 (via (at 133.35 86.106) (size 0.8) (drill 0.4) (layers F.Cu B.Cu) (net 16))
 (segment (start 121.598 87.776) (end 132.95 87.776) (width 0.45) (layer B.Cu) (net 17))
 (segment (start 132.95 87.776) (end 133.35 87.376) (width 0.45) (layer B.Cu) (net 17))
 (segment (start 131.7625 87.376) (end 133.35 87.376) (width 0.45) (layer F.Cu) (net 17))
 (via (at 133.35 87.376) (size 0.8) (drill 0.4) (layers F.Cu B.Cu) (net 17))
 (segment (start 123.831961 89.0905) (end 124.0565 89.0905) (width 0.45) (layer B.Cu) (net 18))
 (segment (start 124.0565 89.0905) (end 125.4125 90.4465) (width 0.45) (layer B.Cu) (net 18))
 (segment (start 123.831961 89.0905) (end 123.831961 84.256039) (width 0.45) (layer F.Cu) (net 18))
 (segment (start 123.831961 84.256039) (end 125.095 82.993) (width 0.45) (layer F.Cu) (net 18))
 (segment (start 128.282 81.756) (end 126.332 81.756) (width 0.45) (layer F.Cu) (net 18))
 (segment (start 126.332 81.756) (end 125.095 82.993) (width 0.45) (layer F.Cu) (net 18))
 (segment (start 125.095 82.993) (end 125.095 82.9945) (width 0.45) (layer F.Cu) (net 18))
 (segment (start 121.598 88.576) (end 123.317461 88.576) (width 0.45) (layer B.Cu) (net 18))
 (via (at 123.831961 89.0905) (size 0.8) (drill 0.4) (layers F.Cu B.Cu) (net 18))
 (segment (start 123.317461 88.576) (end 123.431962 88.690501) (width 0.45) (layer B.Cu) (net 18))
 (segment (start 123.431962 88.690501) (end 123.831961 89.0905) (width 0.45) (layer B.Cu) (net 18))
 (segment (start 110.236 91.778) (end 111.9915 91.778) (width 0.45) (layer B.Cu) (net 26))
 (segment (start 111.9915 91.778) (end 112.395 92.1815) (width 0.45) (layer B.Cu) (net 26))
 (segment (start 112.395 92.1815) (end 112.395 90.879) (width 0.45) (layer B.Cu) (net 26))
 (segment (start 112.395 90.879) (end 113.098 90.176) (width 0.45) (layer B.Cu) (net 26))
 (segment (start 111.76 81.788) (end 108.614 81.788) (width 0.45) (layer F.Cu) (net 32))
 (segment (start 108.614 81.788) (end 108.582 81.756) (width 0.45) (layer F.Cu) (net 32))
 (segment (start 113.098 84.576) (end 113.098 83.126) (width 0.45) (layer B.Cu) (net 32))
 (segment (start 113.098 83.126) (end 111.76 81.788) (width 0.45) (layer B.Cu) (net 32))
 (via (at 111.76 81.788) (size 0.8) (drill 0.4) (layers F.Cu B.Cu) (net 32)))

